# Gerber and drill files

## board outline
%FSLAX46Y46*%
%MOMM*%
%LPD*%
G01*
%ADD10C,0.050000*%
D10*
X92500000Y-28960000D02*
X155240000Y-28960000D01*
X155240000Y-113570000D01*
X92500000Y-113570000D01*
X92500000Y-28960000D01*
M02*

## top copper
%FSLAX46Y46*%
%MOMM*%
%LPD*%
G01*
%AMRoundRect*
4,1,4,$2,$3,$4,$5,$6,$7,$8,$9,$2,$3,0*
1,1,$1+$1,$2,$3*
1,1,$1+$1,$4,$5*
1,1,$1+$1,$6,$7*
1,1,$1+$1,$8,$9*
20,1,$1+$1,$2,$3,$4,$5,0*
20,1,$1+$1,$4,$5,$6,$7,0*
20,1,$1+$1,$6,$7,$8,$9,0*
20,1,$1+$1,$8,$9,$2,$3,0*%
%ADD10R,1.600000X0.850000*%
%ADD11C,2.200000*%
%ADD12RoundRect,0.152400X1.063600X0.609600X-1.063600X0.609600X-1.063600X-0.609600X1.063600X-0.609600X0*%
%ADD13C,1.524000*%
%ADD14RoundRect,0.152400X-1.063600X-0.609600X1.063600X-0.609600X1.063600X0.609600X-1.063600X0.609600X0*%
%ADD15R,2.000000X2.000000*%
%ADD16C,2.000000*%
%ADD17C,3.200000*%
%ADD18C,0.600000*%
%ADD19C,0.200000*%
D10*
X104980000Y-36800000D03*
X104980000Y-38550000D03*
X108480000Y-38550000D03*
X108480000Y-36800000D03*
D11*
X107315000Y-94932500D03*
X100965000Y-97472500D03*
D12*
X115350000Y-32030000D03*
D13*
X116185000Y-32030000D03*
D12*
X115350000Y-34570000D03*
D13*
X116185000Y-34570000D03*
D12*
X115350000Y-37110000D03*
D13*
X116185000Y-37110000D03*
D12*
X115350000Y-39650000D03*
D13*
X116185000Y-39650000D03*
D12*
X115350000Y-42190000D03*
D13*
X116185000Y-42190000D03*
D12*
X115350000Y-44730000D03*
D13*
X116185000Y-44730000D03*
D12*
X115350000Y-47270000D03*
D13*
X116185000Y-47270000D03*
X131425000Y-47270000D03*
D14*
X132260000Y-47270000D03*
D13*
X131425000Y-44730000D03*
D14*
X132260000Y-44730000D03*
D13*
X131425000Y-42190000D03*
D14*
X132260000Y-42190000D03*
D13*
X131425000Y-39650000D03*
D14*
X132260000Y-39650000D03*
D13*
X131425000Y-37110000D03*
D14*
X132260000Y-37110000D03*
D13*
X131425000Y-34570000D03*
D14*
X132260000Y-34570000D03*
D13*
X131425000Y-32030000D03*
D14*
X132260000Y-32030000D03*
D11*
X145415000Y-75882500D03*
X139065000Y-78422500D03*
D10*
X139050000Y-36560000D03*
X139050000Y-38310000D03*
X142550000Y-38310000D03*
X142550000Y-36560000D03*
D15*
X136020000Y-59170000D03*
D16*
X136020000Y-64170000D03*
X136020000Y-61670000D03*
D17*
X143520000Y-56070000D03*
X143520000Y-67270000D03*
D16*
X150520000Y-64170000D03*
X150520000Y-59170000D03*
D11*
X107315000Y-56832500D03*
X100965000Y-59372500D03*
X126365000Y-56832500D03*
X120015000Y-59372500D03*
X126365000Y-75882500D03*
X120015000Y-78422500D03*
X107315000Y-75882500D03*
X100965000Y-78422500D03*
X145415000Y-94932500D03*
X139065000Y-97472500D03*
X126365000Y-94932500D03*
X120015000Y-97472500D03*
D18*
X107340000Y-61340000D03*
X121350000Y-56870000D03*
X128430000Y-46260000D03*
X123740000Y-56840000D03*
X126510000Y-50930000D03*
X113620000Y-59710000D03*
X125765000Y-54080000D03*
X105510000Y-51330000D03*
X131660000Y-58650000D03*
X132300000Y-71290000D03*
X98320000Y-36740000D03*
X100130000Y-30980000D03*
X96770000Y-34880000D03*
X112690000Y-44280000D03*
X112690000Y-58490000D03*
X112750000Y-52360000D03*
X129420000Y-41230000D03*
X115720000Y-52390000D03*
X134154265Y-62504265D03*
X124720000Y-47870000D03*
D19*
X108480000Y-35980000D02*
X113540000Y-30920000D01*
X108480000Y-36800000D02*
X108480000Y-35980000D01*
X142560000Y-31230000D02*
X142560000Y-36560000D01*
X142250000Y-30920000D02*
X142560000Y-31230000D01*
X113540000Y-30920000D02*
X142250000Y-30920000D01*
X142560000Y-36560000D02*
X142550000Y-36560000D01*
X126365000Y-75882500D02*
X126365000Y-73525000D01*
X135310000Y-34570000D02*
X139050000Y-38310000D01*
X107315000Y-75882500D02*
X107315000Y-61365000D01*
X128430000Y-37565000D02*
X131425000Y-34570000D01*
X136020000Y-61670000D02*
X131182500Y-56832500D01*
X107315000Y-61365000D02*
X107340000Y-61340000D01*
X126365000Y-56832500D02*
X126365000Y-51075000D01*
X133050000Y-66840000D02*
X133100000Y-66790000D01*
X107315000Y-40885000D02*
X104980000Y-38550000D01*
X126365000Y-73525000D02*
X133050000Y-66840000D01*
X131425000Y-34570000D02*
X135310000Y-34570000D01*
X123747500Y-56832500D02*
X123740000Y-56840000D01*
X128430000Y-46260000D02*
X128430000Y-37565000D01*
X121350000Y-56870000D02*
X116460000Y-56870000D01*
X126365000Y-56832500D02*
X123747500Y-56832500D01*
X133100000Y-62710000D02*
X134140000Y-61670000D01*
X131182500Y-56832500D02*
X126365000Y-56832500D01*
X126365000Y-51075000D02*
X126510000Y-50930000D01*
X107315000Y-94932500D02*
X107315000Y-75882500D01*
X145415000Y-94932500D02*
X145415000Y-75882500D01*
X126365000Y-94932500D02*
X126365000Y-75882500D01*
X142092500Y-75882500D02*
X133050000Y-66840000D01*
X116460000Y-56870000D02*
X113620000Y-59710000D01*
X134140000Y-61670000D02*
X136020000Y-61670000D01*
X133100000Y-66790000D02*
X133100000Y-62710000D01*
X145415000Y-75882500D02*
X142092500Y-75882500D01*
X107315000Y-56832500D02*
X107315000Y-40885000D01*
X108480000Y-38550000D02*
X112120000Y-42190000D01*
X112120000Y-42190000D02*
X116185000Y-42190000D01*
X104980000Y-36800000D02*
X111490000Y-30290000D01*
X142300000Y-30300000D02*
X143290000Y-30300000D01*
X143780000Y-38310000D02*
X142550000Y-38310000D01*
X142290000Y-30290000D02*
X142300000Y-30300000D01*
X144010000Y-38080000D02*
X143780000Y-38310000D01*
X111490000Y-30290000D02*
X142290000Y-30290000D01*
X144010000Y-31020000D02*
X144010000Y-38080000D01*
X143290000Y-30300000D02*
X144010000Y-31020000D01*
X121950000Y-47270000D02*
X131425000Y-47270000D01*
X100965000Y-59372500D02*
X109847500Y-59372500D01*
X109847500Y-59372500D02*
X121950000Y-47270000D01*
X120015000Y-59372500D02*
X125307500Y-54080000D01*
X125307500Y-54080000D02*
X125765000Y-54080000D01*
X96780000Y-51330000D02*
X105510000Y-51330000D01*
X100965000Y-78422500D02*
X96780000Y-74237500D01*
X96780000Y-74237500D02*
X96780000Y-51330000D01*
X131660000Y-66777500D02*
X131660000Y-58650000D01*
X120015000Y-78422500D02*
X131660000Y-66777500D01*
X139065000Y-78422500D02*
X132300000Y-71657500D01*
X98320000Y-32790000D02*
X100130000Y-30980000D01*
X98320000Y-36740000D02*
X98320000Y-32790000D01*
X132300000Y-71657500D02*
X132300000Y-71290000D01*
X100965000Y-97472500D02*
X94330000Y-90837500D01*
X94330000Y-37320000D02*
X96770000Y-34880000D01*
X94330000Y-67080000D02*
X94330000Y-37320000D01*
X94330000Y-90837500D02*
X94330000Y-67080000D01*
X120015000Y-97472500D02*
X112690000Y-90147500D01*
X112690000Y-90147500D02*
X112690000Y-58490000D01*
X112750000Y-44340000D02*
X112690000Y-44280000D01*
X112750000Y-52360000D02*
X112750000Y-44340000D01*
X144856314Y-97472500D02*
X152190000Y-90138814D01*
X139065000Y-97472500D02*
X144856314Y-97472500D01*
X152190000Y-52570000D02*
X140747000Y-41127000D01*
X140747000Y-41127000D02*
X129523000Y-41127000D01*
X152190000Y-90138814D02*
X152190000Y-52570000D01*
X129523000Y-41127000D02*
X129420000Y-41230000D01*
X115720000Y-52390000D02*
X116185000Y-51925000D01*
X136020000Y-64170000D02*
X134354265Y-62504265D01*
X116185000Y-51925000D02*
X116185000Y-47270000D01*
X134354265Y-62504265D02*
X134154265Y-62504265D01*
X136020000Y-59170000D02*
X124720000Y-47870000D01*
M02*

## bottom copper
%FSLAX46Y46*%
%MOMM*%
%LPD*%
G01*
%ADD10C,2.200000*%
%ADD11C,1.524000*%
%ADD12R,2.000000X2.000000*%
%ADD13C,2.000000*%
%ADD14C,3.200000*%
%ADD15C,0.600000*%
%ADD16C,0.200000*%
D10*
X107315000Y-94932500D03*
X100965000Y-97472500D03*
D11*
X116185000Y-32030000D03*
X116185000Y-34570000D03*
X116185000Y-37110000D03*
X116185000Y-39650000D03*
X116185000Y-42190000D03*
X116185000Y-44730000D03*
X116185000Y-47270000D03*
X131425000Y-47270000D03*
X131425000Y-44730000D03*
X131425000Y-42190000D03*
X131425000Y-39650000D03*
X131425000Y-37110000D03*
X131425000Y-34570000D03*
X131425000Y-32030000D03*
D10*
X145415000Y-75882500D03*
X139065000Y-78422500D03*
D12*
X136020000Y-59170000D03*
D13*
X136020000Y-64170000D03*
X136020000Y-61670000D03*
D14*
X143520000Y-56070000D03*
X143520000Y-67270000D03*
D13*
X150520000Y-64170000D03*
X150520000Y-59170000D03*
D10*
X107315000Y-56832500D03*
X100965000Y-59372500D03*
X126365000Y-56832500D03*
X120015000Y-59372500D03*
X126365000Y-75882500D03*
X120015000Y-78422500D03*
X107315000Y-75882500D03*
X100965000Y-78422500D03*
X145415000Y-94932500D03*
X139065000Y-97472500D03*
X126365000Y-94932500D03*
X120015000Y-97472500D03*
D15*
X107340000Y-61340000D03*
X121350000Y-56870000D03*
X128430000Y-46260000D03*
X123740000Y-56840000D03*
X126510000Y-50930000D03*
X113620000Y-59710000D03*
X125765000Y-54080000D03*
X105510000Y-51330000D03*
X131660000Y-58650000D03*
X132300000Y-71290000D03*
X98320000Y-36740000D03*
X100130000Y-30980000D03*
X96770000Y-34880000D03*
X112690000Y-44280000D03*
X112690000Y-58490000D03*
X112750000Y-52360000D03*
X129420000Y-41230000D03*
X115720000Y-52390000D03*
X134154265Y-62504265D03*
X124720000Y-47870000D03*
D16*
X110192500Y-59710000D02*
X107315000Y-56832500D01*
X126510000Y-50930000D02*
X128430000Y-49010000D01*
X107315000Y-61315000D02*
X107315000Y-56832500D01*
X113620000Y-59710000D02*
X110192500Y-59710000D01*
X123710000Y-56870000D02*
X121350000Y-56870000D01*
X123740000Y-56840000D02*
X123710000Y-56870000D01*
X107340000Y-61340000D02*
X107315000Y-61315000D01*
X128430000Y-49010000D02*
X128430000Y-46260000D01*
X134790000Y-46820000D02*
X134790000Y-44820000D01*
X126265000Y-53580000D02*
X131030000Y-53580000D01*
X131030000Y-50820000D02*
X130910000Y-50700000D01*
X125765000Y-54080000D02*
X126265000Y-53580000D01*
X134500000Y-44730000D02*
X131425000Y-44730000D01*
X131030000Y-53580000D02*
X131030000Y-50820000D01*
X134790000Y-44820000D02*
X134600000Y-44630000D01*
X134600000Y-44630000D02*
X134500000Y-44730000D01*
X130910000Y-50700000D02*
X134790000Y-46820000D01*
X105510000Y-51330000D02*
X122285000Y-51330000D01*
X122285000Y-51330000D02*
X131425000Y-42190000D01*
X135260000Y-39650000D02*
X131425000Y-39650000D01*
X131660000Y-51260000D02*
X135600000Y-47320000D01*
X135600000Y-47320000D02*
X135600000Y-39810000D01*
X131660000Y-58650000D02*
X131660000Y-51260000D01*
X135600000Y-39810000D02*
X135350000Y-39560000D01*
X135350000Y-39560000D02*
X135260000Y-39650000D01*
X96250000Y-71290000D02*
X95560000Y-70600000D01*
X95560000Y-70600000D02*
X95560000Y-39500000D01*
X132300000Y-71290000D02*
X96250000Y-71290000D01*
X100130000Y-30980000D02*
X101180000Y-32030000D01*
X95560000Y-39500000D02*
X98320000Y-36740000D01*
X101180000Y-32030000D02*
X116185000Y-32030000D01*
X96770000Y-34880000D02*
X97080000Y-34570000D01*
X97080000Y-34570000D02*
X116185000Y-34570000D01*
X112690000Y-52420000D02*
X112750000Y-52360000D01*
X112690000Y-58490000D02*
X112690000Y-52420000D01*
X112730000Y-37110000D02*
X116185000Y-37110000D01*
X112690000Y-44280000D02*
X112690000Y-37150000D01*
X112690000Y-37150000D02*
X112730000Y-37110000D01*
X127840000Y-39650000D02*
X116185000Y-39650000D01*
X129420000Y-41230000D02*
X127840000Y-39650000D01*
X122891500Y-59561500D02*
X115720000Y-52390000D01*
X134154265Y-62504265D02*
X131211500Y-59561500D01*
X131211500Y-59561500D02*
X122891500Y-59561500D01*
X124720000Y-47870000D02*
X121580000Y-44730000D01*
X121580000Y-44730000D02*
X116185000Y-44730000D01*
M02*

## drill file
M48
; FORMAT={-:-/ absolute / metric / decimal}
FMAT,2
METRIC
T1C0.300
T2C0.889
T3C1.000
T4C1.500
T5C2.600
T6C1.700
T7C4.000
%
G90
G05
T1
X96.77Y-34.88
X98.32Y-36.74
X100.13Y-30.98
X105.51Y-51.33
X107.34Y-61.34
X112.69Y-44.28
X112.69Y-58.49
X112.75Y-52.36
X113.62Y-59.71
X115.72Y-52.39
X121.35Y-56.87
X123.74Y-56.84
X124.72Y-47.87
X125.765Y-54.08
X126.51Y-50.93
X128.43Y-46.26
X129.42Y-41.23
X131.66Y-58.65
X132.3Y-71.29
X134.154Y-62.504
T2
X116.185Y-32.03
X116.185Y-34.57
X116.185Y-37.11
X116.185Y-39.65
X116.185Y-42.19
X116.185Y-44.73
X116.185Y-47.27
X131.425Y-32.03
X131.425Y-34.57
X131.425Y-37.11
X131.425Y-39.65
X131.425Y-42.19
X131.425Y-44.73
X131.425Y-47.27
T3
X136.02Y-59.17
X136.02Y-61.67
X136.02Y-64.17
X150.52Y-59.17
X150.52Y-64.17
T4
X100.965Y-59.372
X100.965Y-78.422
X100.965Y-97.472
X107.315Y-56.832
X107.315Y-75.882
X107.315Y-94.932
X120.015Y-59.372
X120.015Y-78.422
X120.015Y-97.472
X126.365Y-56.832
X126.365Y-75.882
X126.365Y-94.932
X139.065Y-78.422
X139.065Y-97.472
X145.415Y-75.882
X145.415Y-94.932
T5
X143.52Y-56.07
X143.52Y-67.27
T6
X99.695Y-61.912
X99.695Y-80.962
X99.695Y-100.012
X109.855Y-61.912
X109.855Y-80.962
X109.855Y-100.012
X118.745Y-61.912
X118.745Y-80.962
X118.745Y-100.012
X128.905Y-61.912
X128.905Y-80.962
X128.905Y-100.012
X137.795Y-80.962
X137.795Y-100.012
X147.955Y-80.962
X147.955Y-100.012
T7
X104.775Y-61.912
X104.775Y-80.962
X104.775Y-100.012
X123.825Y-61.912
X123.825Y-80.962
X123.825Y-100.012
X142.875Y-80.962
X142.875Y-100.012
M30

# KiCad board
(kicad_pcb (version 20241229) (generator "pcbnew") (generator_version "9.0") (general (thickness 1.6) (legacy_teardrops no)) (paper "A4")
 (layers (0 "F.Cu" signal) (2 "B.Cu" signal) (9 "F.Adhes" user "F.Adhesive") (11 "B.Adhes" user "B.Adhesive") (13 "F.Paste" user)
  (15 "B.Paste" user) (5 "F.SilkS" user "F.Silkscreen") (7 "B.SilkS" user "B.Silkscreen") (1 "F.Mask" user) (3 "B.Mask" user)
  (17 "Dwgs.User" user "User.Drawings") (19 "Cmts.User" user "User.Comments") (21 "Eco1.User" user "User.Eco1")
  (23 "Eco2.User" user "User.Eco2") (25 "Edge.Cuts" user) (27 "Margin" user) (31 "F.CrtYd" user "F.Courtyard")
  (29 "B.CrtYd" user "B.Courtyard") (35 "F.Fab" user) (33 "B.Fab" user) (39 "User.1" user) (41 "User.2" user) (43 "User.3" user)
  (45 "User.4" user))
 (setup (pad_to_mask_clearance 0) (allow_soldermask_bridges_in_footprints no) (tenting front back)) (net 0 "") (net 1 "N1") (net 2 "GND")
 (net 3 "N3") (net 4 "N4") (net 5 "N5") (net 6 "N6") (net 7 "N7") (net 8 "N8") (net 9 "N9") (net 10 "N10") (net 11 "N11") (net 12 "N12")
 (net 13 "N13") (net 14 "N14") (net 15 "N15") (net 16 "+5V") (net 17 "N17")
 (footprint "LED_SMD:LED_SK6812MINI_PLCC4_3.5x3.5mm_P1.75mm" (layer "F.Cu") (at 106.73 37.675)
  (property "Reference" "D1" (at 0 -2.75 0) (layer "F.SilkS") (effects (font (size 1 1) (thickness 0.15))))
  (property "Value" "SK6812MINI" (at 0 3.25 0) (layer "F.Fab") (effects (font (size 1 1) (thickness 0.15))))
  (pad "1" smd rect (at -1.75 -0.875) (size 1.6 0.85) (layers "F.Cu" "F.Mask" "F.Paste") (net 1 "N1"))
  (pad "2" smd rect (at -1.75 0.875) (size 1.6 0.85) (layers "F.Cu" "F.Mask" "F.Paste") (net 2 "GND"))
  (pad "3" smd rect (at 1.75 0.875) (size 1.6 0.85) (layers "F.Cu" "F.Mask" "F.Paste") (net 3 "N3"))
  (pad "4" smd rect (at 1.75 -0.875) (size 1.6 0.85) (layers "F.Cu" "F.Mask" "F.Paste") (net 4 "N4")))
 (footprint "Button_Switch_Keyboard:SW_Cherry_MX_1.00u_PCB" (layer "F.Cu") (at 107.315 94.9325)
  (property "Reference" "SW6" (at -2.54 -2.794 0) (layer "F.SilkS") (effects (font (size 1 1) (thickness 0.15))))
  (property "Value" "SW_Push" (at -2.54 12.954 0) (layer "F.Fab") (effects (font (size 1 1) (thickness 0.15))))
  (pad "" np_thru_hole circle (at -7.62 5.08) (size 1.7 1.7) (drill 1.7) (layers "*.Cu" "*.Mask"))
  (pad "" np_thru_hole circle (at -2.54 5.08) (size 4 4) (drill 4) (layers "*.Cu" "*.Mask"))
  (pad "" np_thru_hole circle (at 2.54 5.08) (size 1.7 1.7) (drill 1.7) (layers "*.Cu" "*.Mask"))
  (pad "1" thru_hole circle (at 0 0) (size 2.2 2.2) (drill 1.5) (layers "*.Cu" "*.Mask") (remove_unused_layers no) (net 2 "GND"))
  (pad "2" thru_hole circle (at -6.35 2.54) (size 2.2 2.2) (drill 1.5) (layers "*.Cu" "*.Mask") (remove_unused_layers no) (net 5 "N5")))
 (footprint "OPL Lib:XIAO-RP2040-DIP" (layer "F.Cu") (at 123.805 39.65)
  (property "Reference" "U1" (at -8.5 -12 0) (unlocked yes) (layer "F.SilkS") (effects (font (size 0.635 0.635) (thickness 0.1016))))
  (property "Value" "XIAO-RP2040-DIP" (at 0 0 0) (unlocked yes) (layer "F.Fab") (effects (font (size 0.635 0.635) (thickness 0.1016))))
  (pad "1" smd roundrect (at -8.455 -7.62 180) (size 2.432 1.524) (layers "F.Cu" "F.Mask") (roundrect_rratio 0.1) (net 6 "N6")
   (thermal_bridge_angle 45))
  (pad "1" thru_hole circle (at -7.62 -7.62 180) (size 1.524 1.524) (drill 0.889) (layers "*.Cu" "*.Mask") (remove_unused_layers no)
   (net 6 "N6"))
  (pad "2" smd roundrect (at -8.455 -5.08 180) (size 2.432 1.524) (layers "F.Cu" "F.Mask") (roundrect_rratio 0.1) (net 5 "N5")
   (thermal_bridge_angle 45))
  (pad "2" thru_hole circle (at -7.62 -5.08 180) (size 1.524 1.524) (drill 0.889) (layers "*.Cu" "*.Mask") (remove_unused_layers no)
   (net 5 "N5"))
  (pad "3" smd roundrect (at -8.455 -2.54 180) (size 2.432 1.524) (layers "F.Cu" "F.Mask") (roundrect_rratio 0.1) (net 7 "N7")
   (thermal_bridge_angle 45))
  (pad "3" thru_hole circle (at -7.62 -2.54 180) (size 1.524 1.524) (drill 0.889) (layers "*.Cu" "*.Mask") (remove_unused_layers no)
   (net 7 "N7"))
  (pad "4" smd roundrect (at -8.455 0 180) (size 2.432 1.524) (layers "F.Cu" "F.Mask") (roundrect_rratio 0.1) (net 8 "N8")
   (thermal_bridge_angle 45))
  (pad "4" thru_hole circle (at -7.62 0 180) (size 1.524 1.524) (drill 0.889) (layers "*.Cu" "*.Mask") (remove_unused_layers no)
   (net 8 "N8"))
  (pad "5" smd roundrect (at -8.455 2.54 180) (size 2.432 1.524) (layers "F.Cu" "F.Mask") (roundrect_rratio 0.1) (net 3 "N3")
   (thermal_bridge_angle 45))
  (pad "5" thru_hole circle (at -7.62 2.54 180) (size 1.524 1.524) (drill 0.889) (layers "*.Cu" "*.Mask") (remove_unused_layers no)
   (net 3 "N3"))
  (pad "6" smd roundrect (at -8.455 5.08 180) (size 2.432 1.524) (layers "F.Cu" "F.Mask") (roundrect_rratio 0.1) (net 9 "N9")
   (thermal_bridge_angle 45))
  (pad "6" thru_hole circle (at -7.62 5.08 180) (size 1.524 1.524) (drill 0.889) (layers "*.Cu" "*.Mask") (remove_unused_layers no)
   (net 9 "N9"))
  (pad "7" smd roundrect (at -8.455 7.62 180) (size 2.432 1.524) (layers "F.Cu" "F.Mask") (roundrect_rratio 0.1) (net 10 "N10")
   (thermal_bridge_angle 45))
  (pad "7" thru_hole circle (at -7.62 7.62 180) (size 1.524 1.524) (drill 0.889) (layers "*.Cu" "*.Mask") (remove_unused_layers no)
   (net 10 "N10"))
  (pad "8" thru_hole circle (at 7.62 7.62) (size 1.524 1.524) (drill 0.889) (layers "*.Cu" "*.Mask") (remove_unused_layers no)
   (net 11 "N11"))
  (pad "8" smd roundrect (at 8.455 7.62) (size 2.432 1.524) (layers "F.Cu" "F.Mask") (roundrect_rratio 0.1) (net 11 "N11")
   (thermal_bridge_angle 45))
  (pad "9" thru_hole circle (at 7.62 5.08) (size 1.524 1.524) (drill 0.889) (layers "*.Cu" "*.Mask") (remove_unused_layers no)
   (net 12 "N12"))
  (pad "9" smd roundrect (at 8.455 5.08) (size 2.432 1.524) (layers "F.Cu" "F.Mask") (roundrect_rratio 0.1) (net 12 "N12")
   (thermal_bridge_angle 45))
  (pad "10" thru_hole circle (at 7.62 2.54) (size 1.524 1.524) (drill 0.889) (layers "*.Cu" "*.Mask") (remove_unused_layers no)
   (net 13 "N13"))
  (pad "10" smd roundrect (at 8.455 2.54) (size 2.432 1.524) (layers "F.Cu" "F.Mask") (roundrect_rratio 0.1) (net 13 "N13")
   (thermal_bridge_angle 45))
  (pad "11" thru_hole circle (at 7.62 0) (size 1.524 1.524) (drill 0.889) (layers "*.Cu" "*.Mask") (remove_unused_layers no) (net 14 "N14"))
  (pad "11" smd roundrect (at 8.455 0) (size 2.432 1.524) (layers "F.Cu" "F.Mask") (roundrect_rratio 0.1) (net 14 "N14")
   (thermal_bridge_angle 45))
  (pad "12" thru_hole circle (at 7.62 -2.54) (size 1.524 1.524) (drill 0.889) (layers "*.Cu" "*.Mask") (remove_unused_layers no)
   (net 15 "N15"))
  (pad "12" smd roundrect (at 8.455 -2.54) (size 2.432 1.524) (layers "F.Cu" "F.Mask") (roundrect_rratio 0.1) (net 15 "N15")
   (thermal_bridge_angle 45))
  (pad "13" thru_hole circle (at 7.62 -5.08) (size 1.524 1.524) (drill 0.889) (layers "*.Cu" "*.Mask") (remove_unused_layers no)
   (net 2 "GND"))
  (pad "13" smd roundrect (at 8.455 -5.08) (size 2.432 1.524) (layers "F.Cu" "F.Mask") (roundrect_rratio 0.1) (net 2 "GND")
   (thermal_bridge_angle 45))
  (pad "14" thru_hole circle (at 7.62 -7.62) (size 1.524 1.524) (drill 0.889) (layers "*.Cu" "*.Mask") (remove_unused_layers no)
   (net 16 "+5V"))
  (pad "14" smd roundrect (at 8.455 -7.62) (size 2.432 1.524) (layers "F.Cu" "F.Mask") (roundrect_rratio 0.1) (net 16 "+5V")
   (thermal_bridge_angle 45)))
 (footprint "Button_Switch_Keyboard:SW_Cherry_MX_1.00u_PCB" (layer "F.Cu") (at 145.415 75.8825)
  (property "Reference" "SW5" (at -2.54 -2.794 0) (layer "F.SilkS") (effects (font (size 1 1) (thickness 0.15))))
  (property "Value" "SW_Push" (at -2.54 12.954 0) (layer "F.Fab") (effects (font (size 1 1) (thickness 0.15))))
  (pad "" np_thru_hole circle (at -7.62 5.08) (size 1.7 1.7) (drill 1.7) (layers "*.Cu" "*.Mask"))
  (pad "" np_thru_hole circle (at -2.54 5.08) (size 4 4) (drill 4) (layers "*.Cu" "*.Mask"))
  (pad "" np_thru_hole circle (at 2.54 5.08) (size 1.7 1.7) (drill 1.7) (layers "*.Cu" "*.Mask"))
  (pad "1" thru_hole circle (at 0 0) (size 2.2 2.2) (drill 1.5) (layers "*.Cu" "*.Mask") (remove_unused_layers no) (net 2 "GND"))
  (pad "2" thru_hole circle (at -6.35 2.54) (size 2.2 2.2) (drill 1.5) (layers "*.Cu" "*.Mask") (remove_unused_layers no) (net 6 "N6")))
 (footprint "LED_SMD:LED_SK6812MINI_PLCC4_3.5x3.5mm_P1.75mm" (layer "F.Cu") (at 140.8 37.435)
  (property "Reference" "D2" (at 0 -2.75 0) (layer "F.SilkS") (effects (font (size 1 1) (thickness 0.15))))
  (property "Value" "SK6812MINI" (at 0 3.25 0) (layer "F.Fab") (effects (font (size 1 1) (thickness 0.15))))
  (pad "1" smd rect (at -1.75 -0.875) (size 1.6 0.85) (layers "F.Cu" "F.Mask" "F.Paste") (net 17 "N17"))
  (pad "2" smd rect (at -1.75 0.875) (size 1.6 0.85) (layers "F.Cu" "F.Mask" "F.Paste") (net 2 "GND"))
  (pad "3" smd rect (at 1.75 0.875) (size 1.6 0.85) (layers "F.Cu" "F.Mask" "F.Paste") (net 1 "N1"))
  (pad "4" smd rect (at 1.75 -0.875) (size 1.6 0.85) (layers "F.Cu" "F.Mask" "F.Paste") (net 4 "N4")))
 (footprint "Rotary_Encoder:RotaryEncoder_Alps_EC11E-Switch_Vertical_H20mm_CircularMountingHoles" (layer "F.Cu") (at 136.02 59.17)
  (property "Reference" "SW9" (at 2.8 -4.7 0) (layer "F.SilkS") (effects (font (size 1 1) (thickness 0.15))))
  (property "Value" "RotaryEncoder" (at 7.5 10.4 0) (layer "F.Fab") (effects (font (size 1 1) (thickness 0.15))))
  (pad "A" thru_hole rect (at 0 0) (size 2 2) (drill 1) (layers "*.Cu" "*.Mask") (remove_unused_layers no) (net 9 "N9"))
  (pad "B" thru_hole circle (at 0 5) (size 2 2) (drill 1) (layers "*.Cu" "*.Mask") (remove_unused_layers no) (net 10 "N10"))
  (pad "C" thru_hole circle (at 0 2.5) (size 2 2) (drill 1) (layers "*.Cu" "*.Mask") (remove_unused_layers no) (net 2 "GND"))
  (pad "MP" thru_hole circle (at 7.5 -3.1) (size 3.2 3.2) (drill 2.6) (layers "*.Cu" "*.Mask") (remove_unused_layers no))
  (pad "MP" thru_hole circle (at 7.5 8.1) (size 3.2 3.2) (drill 2.6) (layers "*.Cu" "*.Mask") (remove_unused_layers no))
  (pad "S1" thru_hole circle (at 14.5 5) (size 2 2) (drill 1) (layers "*.Cu" "*.Mask") (remove_unused_layers no))
  (pad "S2" thru_hole circle (at 14.5 0) (size 2 2) (drill 1) (layers "*.Cu" "*.Mask") (remove_unused_layers no)))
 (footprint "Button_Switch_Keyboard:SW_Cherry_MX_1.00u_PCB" (layer "F.Cu") (at 107.315 56.8325)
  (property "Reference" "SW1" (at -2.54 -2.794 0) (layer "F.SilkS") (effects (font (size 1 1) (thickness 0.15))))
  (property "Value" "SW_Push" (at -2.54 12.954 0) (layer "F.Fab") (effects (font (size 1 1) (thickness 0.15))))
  (pad "" np_thru_hole circle (at -7.62 5.08) (size 1.7 1.7) (drill 1.7) (layers "*.Cu" "*.Mask"))
  (pad "" np_thru_hole circle (at -2.54 5.08) (size 4 4) (drill 4) (layers "*.Cu" "*.Mask"))
  (pad "" np_thru_hole circle (at 2.54 5.08) (size 1.7 1.7) (drill 1.7) (layers "*.Cu" "*.Mask"))
  (pad "1" thru_hole circle (at 0 0) (size 2.2 2.2) (drill 1.5) (layers "*.Cu" "*.Mask") (remove_unused_layers no) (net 2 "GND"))
  (pad "2" thru_hole circle (at -6.35 2.54) (size 2.2 2.2) (drill 1.5) (layers "*.Cu" "*.Mask") (remove_unused_layers no) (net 11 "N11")))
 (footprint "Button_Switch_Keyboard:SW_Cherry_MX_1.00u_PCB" (layer "F.Cu") (at 126.365 56.8325)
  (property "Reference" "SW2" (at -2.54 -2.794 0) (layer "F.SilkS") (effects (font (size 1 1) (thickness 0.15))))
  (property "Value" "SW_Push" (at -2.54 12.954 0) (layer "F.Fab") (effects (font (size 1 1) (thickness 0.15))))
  (pad "" np_thru_hole circle (at -7.62 5.08) (size 1.7 1.7) (drill 1.7) (layers "*.Cu" "*.Mask"))
  (pad "" np_thru_hole circle (at -2.54 5.08) (size 4 4) (drill 4) (layers "*.Cu" "*.Mask"))
  (pad "" np_thru_hole circle (at 2.54 5.08) (size 1.7 1.7) (drill 1.7) (layers "*.Cu" "*.Mask"))
  (pad "1" thru_hole circle (at 0 0) (size 2.2 2.2) (drill 1.5) (layers "*.Cu" "*.Mask") (remove_unused_layers no) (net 2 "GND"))
  (pad "2" thru_hole circle (at -6.35 2.54) (size 2.2 2.2) (drill 1.5) (layers "*.Cu" "*.Mask") (remove_unused_layers no) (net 12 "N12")))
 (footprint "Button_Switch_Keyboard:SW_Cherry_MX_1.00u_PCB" (layer "F.Cu") (at 126.365 75.8825)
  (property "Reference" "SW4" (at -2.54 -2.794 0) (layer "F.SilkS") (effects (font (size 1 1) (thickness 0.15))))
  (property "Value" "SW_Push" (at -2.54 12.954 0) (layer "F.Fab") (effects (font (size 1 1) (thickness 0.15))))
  (pad "" np_thru_hole circle (at -7.62 5.08) (size 1.7 1.7) (drill 1.7) (layers "*.Cu" "*.Mask"))
  (pad "" np_thru_hole circle (at -2.54 5.08) (size 4 4) (drill 4) (layers "*.Cu" "*.Mask"))
  (pad "" np_thru_hole circle (at 2.54 5.08) (size 1.7 1.7) (drill 1.7) (layers "*.Cu" "*.Mask"))
  (pad "1" thru_hole circle (at 0 0) (size 2.2 2.2) (drill 1.5) (layers "*.Cu" "*.Mask") (remove_unused_layers no) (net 2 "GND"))
  (pad "2" thru_hole circle (at -6.35 2.54) (size 2.2 2.2) (drill 1.5) (layers "*.Cu" "*.Mask") (remove_unused_layers no) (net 14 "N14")))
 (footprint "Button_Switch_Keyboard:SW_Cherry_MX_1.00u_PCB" (layer "F.Cu") (at 107.315 75.8825)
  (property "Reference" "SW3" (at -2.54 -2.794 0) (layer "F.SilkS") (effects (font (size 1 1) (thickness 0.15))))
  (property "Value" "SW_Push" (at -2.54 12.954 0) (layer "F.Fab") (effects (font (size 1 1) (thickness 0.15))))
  (pad "" np_thru_hole circle (at -7.62 5.08) (size 1.7 1.7) (drill 1.7) (layers "*.Cu" "*.Mask"))
  (pad "" np_thru_hole circle (at -2.54 5.08) (size 4 4) (drill 4) (layers "*.Cu" "*.Mask"))
  (pad "" np_thru_hole circle (at 2.54 5.08) (size 1.7 1.7) (drill 1.7) (layers "*.Cu" "*.Mask"))
  (pad "1" thru_hole circle (at 0 0) (size 2.2 2.2) (drill 1.5) (layers "*.Cu" "*.Mask") (remove_unused_layers no) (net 2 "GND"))
  (pad "2" thru_hole circle (at -6.35 2.54) (size 2.2 2.2) (drill 1.5) (layers "*.Cu" "*.Mask") (remove_unused_layers no) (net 13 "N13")))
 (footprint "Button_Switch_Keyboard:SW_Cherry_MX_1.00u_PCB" (layer "F.Cu") (at 145.415 94.9325)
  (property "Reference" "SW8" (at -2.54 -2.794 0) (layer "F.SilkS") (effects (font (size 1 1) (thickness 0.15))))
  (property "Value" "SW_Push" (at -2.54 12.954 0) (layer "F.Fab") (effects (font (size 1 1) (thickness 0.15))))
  (pad "" np_thru_hole circle (at -7.62 5.08) (size 1.7 1.7) (drill 1.7) (layers "*.Cu" "*.Mask"))
  (pad "" np_thru_hole circle (at -2.54 5.08) (size 4 4) (drill 4) (layers "*.Cu" "*.Mask"))
  (pad "" np_thru_hole circle (at 2.54 5.08) (size 1.7 1.7) (drill 1.7) (layers "*.Cu" "*.Mask"))
  (pad "1" thru_hole circle (at 0 0) (size 2.2 2.2) (drill 1.5) (layers "*.Cu" "*.Mask") (remove_unused_layers no) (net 2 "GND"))
  (pad "2" thru_hole circle (at -6.35 2.54) (size 2.2 2.2) (drill 1.5) (layers "*.Cu" "*.Mask") (remove_unused_layers no) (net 8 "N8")))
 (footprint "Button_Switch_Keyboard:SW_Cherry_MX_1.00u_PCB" (layer "F.Cu") (at 126.365 94.9325)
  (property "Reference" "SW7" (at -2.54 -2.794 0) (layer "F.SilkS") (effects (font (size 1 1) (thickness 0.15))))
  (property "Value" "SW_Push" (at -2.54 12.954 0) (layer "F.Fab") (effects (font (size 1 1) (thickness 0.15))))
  (pad "" np_thru_hole circle (at -7.62 5.08) (size 1.7 1.7) (drill 1.7) (layers "*.Cu" "*.Mask"))
  (pad "" np_thru_hole circle (at -2.54 5.08) (size 4 4) (drill 4) (layers "*.Cu" "*.Mask"))
  (pad "" np_thru_hole circle (at 2.54 5.08) (size 1.7 1.7) (drill 1.7) (layers "*.Cu" "*.Mask"))
  (pad "1" thru_hole circle (at 0 0) (size 2.2 2.2) (drill 1.5) (layers "*.Cu" "*.Mask") (remove_unused_layers no) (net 2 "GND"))
  (pad "2" thru_hole circle (at -6.35 2.54) (size 2.2 2.2) (drill 1.5) (layers "*.Cu" "*.Mask") (remove_unused_layers no) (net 7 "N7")))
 (gr_rect (start 92.5 28.96) (end 155.24 113.57) (stroke (width 0.05) (type default)) (fill no) (layer "Edge.Cuts"))
 (segment (start 108.48 35.98) (end 113.54 30.92) (width 0.2) (layer "F.Cu") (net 4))
 (segment (start 108.48 36.8) (end 108.48 35.98) (width 0.2) (layer "F.Cu") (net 4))
 (segment (start 142.56 31.23) (end 142.56 36.56) (width 0.2) (layer "F.Cu") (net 4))
 (segment (start 142.25 30.92) (end 142.56 31.23) (width 0.2) (layer "F.Cu") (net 4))
 (segment (start 113.54 30.92) (end 142.25 30.92) (width 0.2) (layer "F.Cu") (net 4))
 (segment (start 142.56 36.56) (end 142.55 36.56) (width 0.2) (layer "F.Cu") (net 4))
 (segment (start 126.365 75.8825) (end 126.365 73.525) (width 0.2) (layer "F.Cu") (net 2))
 (segment (start 135.31 34.57) (end 139.05 38.31) (width 0.2) (layer "F.Cu") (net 2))
 (segment (start 107.315 75.8825) (end 107.315 61.365) (width 0.2) (layer "F.Cu") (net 2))
 (segment (start 128.43 37.565) (end 131.425 34.57) (width 0.2) (layer "F.Cu") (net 2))
 (segment (start 136.02 61.67) (end 131.1825 56.8325) (width 0.2) (layer "F.Cu") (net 2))
 (segment (start 107.315 61.365) (end 107.34 61.34) (width 0.2) (layer "F.Cu") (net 2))
 (segment (start 126.365 56.8325) (end 126.365 51.075) (width 0.2) (layer "F.Cu") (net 2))
 (segment (start 133.05 66.84) (end 133.1 66.79) (width 0.2) (layer "F.Cu") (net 2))
 (segment (start 107.315 40.885) (end 104.98 38.55) (width 0.2) (layer "F.Cu") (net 2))
 (segment (start 126.365 73.525) (end 133.05 66.84) (width 0.2) (layer "F.Cu") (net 2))
 (segment (start 131.425 34.57) (end 135.31 34.57) (width 0.2) (layer "F.Cu") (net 2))
 (segment (start 123.7475 56.8325) (end 123.74 56.84) (width 0.2) (layer "F.Cu") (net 2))
 (segment (start 128.43 46.26) (end 128.43 37.565) (width 0.2) (layer "F.Cu") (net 2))
 (segment (start 121.35 56.87) (end 116.46 56.87) (width 0.2) (layer "F.Cu") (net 2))
 (segment (start 126.365 56.8325) (end 123.7475 56.8325) (width 0.2) (layer "F.Cu") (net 2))
 (segment (start 133.1 62.71) (end 134.14 61.67) (width 0.2) (layer "F.Cu") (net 2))
 (segment (start 131.1825 56.8325) (end 126.365 56.8325) (width 0.2) (layer "F.Cu") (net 2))
 (segment (start 126.365 51.075) (end 126.51 50.93) (width 0.2) (layer "F.Cu") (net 2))
 (segment (start 107.315 94.9325) (end 107.315 75.8825) (width 0.2) (layer "F.Cu") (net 2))
 (segment (start 145.415 94.9325) (end 145.415 75.8825) (width 0.2) (layer "F.Cu") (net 2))
 (segment (start 126.365 94.9325) (end 126.365 75.8825) (width 0.2) (layer "F.Cu") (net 2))
 (segment (start 142.0925 75.8825) (end 133.05 66.84) (width 0.2) (layer "F.Cu") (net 2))
 (segment (start 116.46 56.87) (end 113.62 59.71) (width 0.2) (layer "F.Cu") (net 2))
 (segment (start 134.14 61.67) (end 136.02 61.67) (width 0.2) (layer "F.Cu") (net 2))
 (segment (start 133.1 66.79) (end 133.1 62.71) (width 0.2) (layer "F.Cu") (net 2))
 (segment (start 145.415 75.8825) (end 142.0925 75.8825) (width 0.2) (layer "F.Cu") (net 2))
 (segment (start 107.315 56.8325) (end 107.315 40.885) (width 0.2) (layer "F.Cu") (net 2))
 (via (at 107.34 61.34) (size 0.6) (drill 0.3) (layers "F.Cu" "B.Cu") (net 2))
 (via (at 121.35 56.87) (size 0.6) (drill 0.3) (layers "F.Cu" "B.Cu") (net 2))
 (via (at 128.43 46.26) (size 0.6) (drill 0.3) (layers "F.Cu" "B.Cu") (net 2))
 (via (at 123.74 56.84) (size 0.6) (drill 0.3) (layers "F.Cu" "B.Cu") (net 2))
 (via (at 126.51 50.93) (size 0.6) (drill 0.3) (layers "F.Cu" "B.Cu") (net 2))
 (via (at 113.62 59.71) (size 0.6) (drill 0.3) (layers "F.Cu" "B.Cu") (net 2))
 (segment (start 110.1925 59.71) (end 107.315 56.8325) (width 0.2) (layer "B.Cu") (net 2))
 (segment (start 126.51 50.93) (end 128.43 49.01) (width 0.2) (layer "B.Cu") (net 2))
 (segment (start 107.315 61.315) (end 107.315 56.8325) (width 0.2) (layer "B.Cu") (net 2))
 (segment (start 113.62 59.71) (end 110.1925 59.71) (width 0.2) (layer "B.Cu") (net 2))
 (segment (start 123.71 56.87) (end 121.35 56.87) (width 0.2) (layer "B.Cu") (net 2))
 (segment (start 123.74 56.84) (end 123.71 56.87) (width 0.2) (layer "B.Cu") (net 2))
 (segment (start 107.34 61.34) (end 107.315 61.315) (width 0.2) (layer "B.Cu") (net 2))
 (segment (start 128.43 49.01) (end 128.43 46.26) (width 0.2) (layer "B.Cu") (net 2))
 (segment (start 108.48 38.55) (end 112.12 42.19) (width 0.2) (layer "F.Cu") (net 3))
 (segment (start 112.12 42.19) (end 116.185 42.19) (width 0.2) (layer "F.Cu") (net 3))
 (segment (start 104.98 36.8) (end 111.49 30.29) (width 0.2) (layer "F.Cu") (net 1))
 (segment (start 142.3 30.3) (end 143.29 30.3) (width 0.2) (layer "F.Cu") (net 1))
 (segment (start 143.78 38.31) (end 142.55 38.31) (width 0.2) (layer "F.Cu") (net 1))
 (segment (start 142.29 30.29) (end 142.3 30.3) (width 0.2) (layer "F.Cu") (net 1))
 (segment (start 144.01 38.08) (end 143.78 38.31) (width 0.2) (layer "F.Cu") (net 1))
 (segment (start 111.49 30.29) (end 142.29 30.29) (width 0.2) (layer "F.Cu") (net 1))
 (segment (start 144.01 31.02) (end 144.01 38.08) (width 0.2) (layer "F.Cu") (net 1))
 (segment (start 143.29 30.3) (end 144.01 31.02) (width 0.2) (layer "F.Cu") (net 1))
 (segment (start 121.95 47.27) (end 131.425 47.27) (width 0.2) (layer "F.Cu") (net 11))
 (segment (start 100.965 59.3725) (end 109.8475 59.3725) (width 0.2) (layer "F.Cu") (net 11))
 (segment (start 109.8475 59.3725) (end 121.95 47.27) (width 0.2) (layer "F.Cu") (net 11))
 (segment (start 120.015 59.3725) (end 125.3075 54.08) (width 0.2) (layer "F.Cu") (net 12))
 (segment (start 125.3075 54.08) (end 125.765 54.08) (width 0.2) (layer "F.Cu") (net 12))
 (via (at 125.765 54.08) (size 0.6) (drill 0.3) (layers "F.Cu" "B.Cu") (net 12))
 (segment (start 134.79 46.82) (end 134.79 44.82) (width 0.2) (layer "B.Cu") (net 12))
 (segment (start 126.265 53.58) (end 131.03 53.58) (width 0.2) (layer "B.Cu") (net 12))
 (segment (start 131.03 50.82) (end 130.91 50.7) (width 0.2) (layer "B.Cu") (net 12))
 (segment (start 125.765 54.08) (end 126.265 53.58) (width 0.2) (layer "B.Cu") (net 12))
 (segment (start 134.5 44.73) (end 131.425 44.73) (width 0.2) (layer "B.Cu") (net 12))
 (segment (start 131.03 53.58) (end 131.03 50.82) (width 0.2) (layer "B.Cu") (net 12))
 (segment (start 134.79 44.82) (end 134.6 44.63) (width 0.2) (layer "B.Cu") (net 12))
 (segment (start 134.6 44.63) (end 134.5 44.73) (width 0.2) (layer "B.Cu") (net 12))
 (segment (start 130.91 50.7) (end 134.79 46.82) (width 0.2) (layer "B.Cu") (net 12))
 (segment (start 96.78 51.33) (end 105.51 51.33) (width 0.2) (layer "F.Cu") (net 13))
 (segment (start 100.965 78.4225) (end 96.78 74.2375) (width 0.2) (layer "F.Cu") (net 13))
 (segment (start 96.78 74.2375) (end 96.78 51.33) (width 0.2) (layer "F.Cu") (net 13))
 (via (at 105.51 51.33) (size 0.6) (drill 0.3) (layers "F.Cu" "B.Cu") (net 13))
 (segment (start 105.51 51.33) (end 122.285 51.33) (width 0.2) (layer "B.Cu") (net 13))
 (segment (start 122.285 51.33) (end 131.425 42.19) (width 0.2) (layer "B.Cu") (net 13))
 (segment (start 131.66 66.7775) (end 131.66 58.65) (width 0.2) (layer "F.Cu") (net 14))
 (segment (start 120.015 78.4225) (end 131.66 66.7775) (width 0.2) (layer "F.Cu") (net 14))
 (via (at 131.66 58.65) (size 0.6) (drill 0.3) (layers "F.Cu" "B.Cu") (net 14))
 (segment (start 135.26 39.65) (end 131.425 39.65) (width 0.2) (layer "B.Cu") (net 14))
 (segment (start 131.66 51.26) (end 135.6 47.32) (width 0.2) (layer "B.Cu") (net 14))
 (segment (start 135.6 47.32) (end 135.6 39.81) (width 0.2) (layer "B.Cu") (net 14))
 (segment (start 131.66 58.65) (end 131.66 51.26) (width 0.2) (layer "B.Cu") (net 14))
 (segment (start 135.6 39.81) (end 135.35 39.56) (width 0.2) (layer "B.Cu") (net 14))
 (segment (start 135.35 39.56) (end 135.26 39.65) (width 0.2) (layer "B.Cu") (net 14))
 (segment (start 139.065 78.4225) (end 132.3 71.6575) (width 0.2) (layer "F.Cu") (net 6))
 (segment (start 98.32 32.79) (end 100.13 30.98) (width 0.2) (layer "F.Cu") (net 6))
 (segment (start 98.32 36.74) (end 98.32 32.79) (width 0.2) (layer "F.Cu") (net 6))
 (segment (start 132.3 71.6575) (end 132.3 71.29) (width 0.2) (layer "F.Cu") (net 6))
 (via (at 132.3 71.29) (size 0.6) (drill 0.3) (layers "F.Cu" "B.Cu") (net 6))
 (via (at 98.32 36.74) (size 0.6) (drill 0.3) (layers "F.Cu" "B.Cu") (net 6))
 (via (at 100.13 30.98) (size 0.6) (drill 0.3) (layers "F.Cu" "B.Cu") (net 6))
 (segment (start 96.25 71.29) (end 95.56 70.6) (width 0.2) (layer "B.Cu") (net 6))
 (segment (start 95.56 70.6) (end 95.56 39.5) (width 0.2) (layer "B.Cu") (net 6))
 (segment (start 132.3 71.29) (end 96.25 71.29) (width 0.2) (layer "B.Cu") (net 6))
 (segment (start 100.13 30.98) (end 101.18 32.03) (width 0.2) (layer "B.Cu") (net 6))
 (segment (start 95.56 39.5) (end 98.32 36.74) (width 0.2) (layer "B.Cu") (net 6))
 (segment (start 101.18 32.03) (end 116.185 32.03) (width 0.2) (layer "B.Cu") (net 6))
 (segment (start 100.965 97.4725) (end 94.33 90.8375) (width 0.2) (layer "F.Cu") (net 5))
 (segment (start 94.33 37.32) (end 96.77 34.88) (width 0.2) (layer "F.Cu") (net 5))
 (segment (start 94.33 67.08) (end 94.33 37.32) (width 0.2) (layer "F.Cu") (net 5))
 (segment (start 94.33 90.8375) (end 94.33 67.08) (width 0.2) (layer "F.Cu") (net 5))
 (via (at 96.77 34.88) (size 0.6) (drill 0.3) (layers "F.Cu" "B.Cu") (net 5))
 (segment (start 96.77 34.88) (end 97.08 34.57) (width 0.2) (layer "B.Cu") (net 5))
 (segment (start 97.08 34.57) (end 116.185 34.57) (width 0.2) (layer "B.Cu") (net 5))
 (segment (start 120.015 97.4725) (end 112.69 90.1475) (width 0.2) (layer "F.Cu") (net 7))
 (segment (start 112.69 90.1475) (end 112.69 58.49) (width 0.2) (layer "F.Cu") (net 7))
 (segment (start 112.75 44.34) (end 112.69 44.28) (width 0.2) (layer "F.Cu") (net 7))
 (segment (start 112.75 52.36) (end 112.75 44.34) (width 0.2) (layer "F.Cu") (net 7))
 (via (at 112.69 44.28) (size 0.6) (drill 0.3) (layers "F.Cu" "B.Cu") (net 7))
 (via (at 112.69 58.49) (size 0.6) (drill 0.3) (layers "F.Cu" "B.Cu") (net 7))
 (via (at 112.75 52.36) (size 0.6) (drill 0.3) (layers "F.Cu" "B.Cu") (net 7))
 (segment (start 112.69 52.42) (end 112.75 52.36) (width 0.2) (layer "B.Cu") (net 7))
 (segment (start 112.69 58.49) (end 112.69 52.42) (width 0.2) (layer "B.Cu") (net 7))
 (segment (start 112.73 37.11) (end 116.185 37.11) (width 0.2) (layer "B.Cu") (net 7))
 (segment (start 112.69 44.28) (end 112.69 37.15) (width 0.2) (layer "B.Cu") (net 7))
 (segment (start 112.69 37.15) (end 112.73 37.11) (width 0.2) (layer "B.Cu") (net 7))
 (segment (start 144.856314 97.4725) (end 152.19 90.138814) (width 0.2) (layer "F.Cu") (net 8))
 (segment (start 139.065 97.4725) (end 144.856314 97.4725) (width 0.2) (layer "F.Cu") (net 8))
 (segment (start 152.19 52.57) (end 140.747 41.127) (width 0.2) (layer "F.Cu") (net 8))
 (segment (start 140.747 41.127) (end 129.523 41.127) (width 0.2) (layer "F.Cu") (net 8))
 (segment (start 152.19 90.138814) (end 152.19 52.57) (width 0.2) (layer "F.Cu") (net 8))
 (segment (start 129.523 41.127) (end 129.42 41.23) (width 0.2) (layer "F.Cu") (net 8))
 (via (at 129.42 41.23) (size 0.6) (drill 0.3) (layers "F.Cu" "B.Cu") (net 8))
 (segment (start 127.84 39.65) (end 116.185 39.65) (width 0.2) (layer "B.Cu") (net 8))
 (segment (start 129.42 41.23) (end 127.84 39.65) (width 0.2) (layer "B.Cu") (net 8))
 (segment (start 115.72 52.39) (end 116.185 51.925) (width 0.2) (layer "F.Cu") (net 10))
 (segment (start 136.02 64.17) (end 134.354265 62.504265) (width 0.2) (layer "F.Cu") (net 10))
 (segment (start 116.185 51.925) (end 116.185 47.27) (width 0.2) (layer "F.Cu") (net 10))
 (segment (start 134.354265 62.504265) (end 134.154265 62.504265) (width 0.2) (layer "F.Cu") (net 10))
 (via (at 115.72 52.39) (size 0.6) (drill 0.3) (layers "F.Cu" "B.Cu") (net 10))
 (via (at 134.154265 62.504265) (size 0.6) (drill 0.3) (layers "F.Cu" "B.Cu") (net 10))
 (segment (start 122.8915 59.5615) (end 115.72 52.39) (width 0.2) (layer "B.Cu") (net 10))
 (segment (start 134.154265 62.504265) (end 131.2115 59.5615) (width 0.2) (layer "B.Cu") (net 10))
 (segment (start 131.2115 59.5615) (end 122.8915 59.5615) (width 0.2) (layer "B.Cu") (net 10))
 (segment (start 136.02 59.17) (end 124.72 47.87) (width 0.2) (layer "F.Cu") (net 9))
 (via (at 124.72 47.87) (size 0.6) (drill 0.3) (layers "F.Cu" "B.Cu") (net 9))
 (segment (start 124.72 47.87) (end 121.58 44.73) (width 0.2) (layer "B.Cu") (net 9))
 (segment (start 121.58 44.73) (end 116.185 44.73) (width 0.2) (layer "B.Cu") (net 9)))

